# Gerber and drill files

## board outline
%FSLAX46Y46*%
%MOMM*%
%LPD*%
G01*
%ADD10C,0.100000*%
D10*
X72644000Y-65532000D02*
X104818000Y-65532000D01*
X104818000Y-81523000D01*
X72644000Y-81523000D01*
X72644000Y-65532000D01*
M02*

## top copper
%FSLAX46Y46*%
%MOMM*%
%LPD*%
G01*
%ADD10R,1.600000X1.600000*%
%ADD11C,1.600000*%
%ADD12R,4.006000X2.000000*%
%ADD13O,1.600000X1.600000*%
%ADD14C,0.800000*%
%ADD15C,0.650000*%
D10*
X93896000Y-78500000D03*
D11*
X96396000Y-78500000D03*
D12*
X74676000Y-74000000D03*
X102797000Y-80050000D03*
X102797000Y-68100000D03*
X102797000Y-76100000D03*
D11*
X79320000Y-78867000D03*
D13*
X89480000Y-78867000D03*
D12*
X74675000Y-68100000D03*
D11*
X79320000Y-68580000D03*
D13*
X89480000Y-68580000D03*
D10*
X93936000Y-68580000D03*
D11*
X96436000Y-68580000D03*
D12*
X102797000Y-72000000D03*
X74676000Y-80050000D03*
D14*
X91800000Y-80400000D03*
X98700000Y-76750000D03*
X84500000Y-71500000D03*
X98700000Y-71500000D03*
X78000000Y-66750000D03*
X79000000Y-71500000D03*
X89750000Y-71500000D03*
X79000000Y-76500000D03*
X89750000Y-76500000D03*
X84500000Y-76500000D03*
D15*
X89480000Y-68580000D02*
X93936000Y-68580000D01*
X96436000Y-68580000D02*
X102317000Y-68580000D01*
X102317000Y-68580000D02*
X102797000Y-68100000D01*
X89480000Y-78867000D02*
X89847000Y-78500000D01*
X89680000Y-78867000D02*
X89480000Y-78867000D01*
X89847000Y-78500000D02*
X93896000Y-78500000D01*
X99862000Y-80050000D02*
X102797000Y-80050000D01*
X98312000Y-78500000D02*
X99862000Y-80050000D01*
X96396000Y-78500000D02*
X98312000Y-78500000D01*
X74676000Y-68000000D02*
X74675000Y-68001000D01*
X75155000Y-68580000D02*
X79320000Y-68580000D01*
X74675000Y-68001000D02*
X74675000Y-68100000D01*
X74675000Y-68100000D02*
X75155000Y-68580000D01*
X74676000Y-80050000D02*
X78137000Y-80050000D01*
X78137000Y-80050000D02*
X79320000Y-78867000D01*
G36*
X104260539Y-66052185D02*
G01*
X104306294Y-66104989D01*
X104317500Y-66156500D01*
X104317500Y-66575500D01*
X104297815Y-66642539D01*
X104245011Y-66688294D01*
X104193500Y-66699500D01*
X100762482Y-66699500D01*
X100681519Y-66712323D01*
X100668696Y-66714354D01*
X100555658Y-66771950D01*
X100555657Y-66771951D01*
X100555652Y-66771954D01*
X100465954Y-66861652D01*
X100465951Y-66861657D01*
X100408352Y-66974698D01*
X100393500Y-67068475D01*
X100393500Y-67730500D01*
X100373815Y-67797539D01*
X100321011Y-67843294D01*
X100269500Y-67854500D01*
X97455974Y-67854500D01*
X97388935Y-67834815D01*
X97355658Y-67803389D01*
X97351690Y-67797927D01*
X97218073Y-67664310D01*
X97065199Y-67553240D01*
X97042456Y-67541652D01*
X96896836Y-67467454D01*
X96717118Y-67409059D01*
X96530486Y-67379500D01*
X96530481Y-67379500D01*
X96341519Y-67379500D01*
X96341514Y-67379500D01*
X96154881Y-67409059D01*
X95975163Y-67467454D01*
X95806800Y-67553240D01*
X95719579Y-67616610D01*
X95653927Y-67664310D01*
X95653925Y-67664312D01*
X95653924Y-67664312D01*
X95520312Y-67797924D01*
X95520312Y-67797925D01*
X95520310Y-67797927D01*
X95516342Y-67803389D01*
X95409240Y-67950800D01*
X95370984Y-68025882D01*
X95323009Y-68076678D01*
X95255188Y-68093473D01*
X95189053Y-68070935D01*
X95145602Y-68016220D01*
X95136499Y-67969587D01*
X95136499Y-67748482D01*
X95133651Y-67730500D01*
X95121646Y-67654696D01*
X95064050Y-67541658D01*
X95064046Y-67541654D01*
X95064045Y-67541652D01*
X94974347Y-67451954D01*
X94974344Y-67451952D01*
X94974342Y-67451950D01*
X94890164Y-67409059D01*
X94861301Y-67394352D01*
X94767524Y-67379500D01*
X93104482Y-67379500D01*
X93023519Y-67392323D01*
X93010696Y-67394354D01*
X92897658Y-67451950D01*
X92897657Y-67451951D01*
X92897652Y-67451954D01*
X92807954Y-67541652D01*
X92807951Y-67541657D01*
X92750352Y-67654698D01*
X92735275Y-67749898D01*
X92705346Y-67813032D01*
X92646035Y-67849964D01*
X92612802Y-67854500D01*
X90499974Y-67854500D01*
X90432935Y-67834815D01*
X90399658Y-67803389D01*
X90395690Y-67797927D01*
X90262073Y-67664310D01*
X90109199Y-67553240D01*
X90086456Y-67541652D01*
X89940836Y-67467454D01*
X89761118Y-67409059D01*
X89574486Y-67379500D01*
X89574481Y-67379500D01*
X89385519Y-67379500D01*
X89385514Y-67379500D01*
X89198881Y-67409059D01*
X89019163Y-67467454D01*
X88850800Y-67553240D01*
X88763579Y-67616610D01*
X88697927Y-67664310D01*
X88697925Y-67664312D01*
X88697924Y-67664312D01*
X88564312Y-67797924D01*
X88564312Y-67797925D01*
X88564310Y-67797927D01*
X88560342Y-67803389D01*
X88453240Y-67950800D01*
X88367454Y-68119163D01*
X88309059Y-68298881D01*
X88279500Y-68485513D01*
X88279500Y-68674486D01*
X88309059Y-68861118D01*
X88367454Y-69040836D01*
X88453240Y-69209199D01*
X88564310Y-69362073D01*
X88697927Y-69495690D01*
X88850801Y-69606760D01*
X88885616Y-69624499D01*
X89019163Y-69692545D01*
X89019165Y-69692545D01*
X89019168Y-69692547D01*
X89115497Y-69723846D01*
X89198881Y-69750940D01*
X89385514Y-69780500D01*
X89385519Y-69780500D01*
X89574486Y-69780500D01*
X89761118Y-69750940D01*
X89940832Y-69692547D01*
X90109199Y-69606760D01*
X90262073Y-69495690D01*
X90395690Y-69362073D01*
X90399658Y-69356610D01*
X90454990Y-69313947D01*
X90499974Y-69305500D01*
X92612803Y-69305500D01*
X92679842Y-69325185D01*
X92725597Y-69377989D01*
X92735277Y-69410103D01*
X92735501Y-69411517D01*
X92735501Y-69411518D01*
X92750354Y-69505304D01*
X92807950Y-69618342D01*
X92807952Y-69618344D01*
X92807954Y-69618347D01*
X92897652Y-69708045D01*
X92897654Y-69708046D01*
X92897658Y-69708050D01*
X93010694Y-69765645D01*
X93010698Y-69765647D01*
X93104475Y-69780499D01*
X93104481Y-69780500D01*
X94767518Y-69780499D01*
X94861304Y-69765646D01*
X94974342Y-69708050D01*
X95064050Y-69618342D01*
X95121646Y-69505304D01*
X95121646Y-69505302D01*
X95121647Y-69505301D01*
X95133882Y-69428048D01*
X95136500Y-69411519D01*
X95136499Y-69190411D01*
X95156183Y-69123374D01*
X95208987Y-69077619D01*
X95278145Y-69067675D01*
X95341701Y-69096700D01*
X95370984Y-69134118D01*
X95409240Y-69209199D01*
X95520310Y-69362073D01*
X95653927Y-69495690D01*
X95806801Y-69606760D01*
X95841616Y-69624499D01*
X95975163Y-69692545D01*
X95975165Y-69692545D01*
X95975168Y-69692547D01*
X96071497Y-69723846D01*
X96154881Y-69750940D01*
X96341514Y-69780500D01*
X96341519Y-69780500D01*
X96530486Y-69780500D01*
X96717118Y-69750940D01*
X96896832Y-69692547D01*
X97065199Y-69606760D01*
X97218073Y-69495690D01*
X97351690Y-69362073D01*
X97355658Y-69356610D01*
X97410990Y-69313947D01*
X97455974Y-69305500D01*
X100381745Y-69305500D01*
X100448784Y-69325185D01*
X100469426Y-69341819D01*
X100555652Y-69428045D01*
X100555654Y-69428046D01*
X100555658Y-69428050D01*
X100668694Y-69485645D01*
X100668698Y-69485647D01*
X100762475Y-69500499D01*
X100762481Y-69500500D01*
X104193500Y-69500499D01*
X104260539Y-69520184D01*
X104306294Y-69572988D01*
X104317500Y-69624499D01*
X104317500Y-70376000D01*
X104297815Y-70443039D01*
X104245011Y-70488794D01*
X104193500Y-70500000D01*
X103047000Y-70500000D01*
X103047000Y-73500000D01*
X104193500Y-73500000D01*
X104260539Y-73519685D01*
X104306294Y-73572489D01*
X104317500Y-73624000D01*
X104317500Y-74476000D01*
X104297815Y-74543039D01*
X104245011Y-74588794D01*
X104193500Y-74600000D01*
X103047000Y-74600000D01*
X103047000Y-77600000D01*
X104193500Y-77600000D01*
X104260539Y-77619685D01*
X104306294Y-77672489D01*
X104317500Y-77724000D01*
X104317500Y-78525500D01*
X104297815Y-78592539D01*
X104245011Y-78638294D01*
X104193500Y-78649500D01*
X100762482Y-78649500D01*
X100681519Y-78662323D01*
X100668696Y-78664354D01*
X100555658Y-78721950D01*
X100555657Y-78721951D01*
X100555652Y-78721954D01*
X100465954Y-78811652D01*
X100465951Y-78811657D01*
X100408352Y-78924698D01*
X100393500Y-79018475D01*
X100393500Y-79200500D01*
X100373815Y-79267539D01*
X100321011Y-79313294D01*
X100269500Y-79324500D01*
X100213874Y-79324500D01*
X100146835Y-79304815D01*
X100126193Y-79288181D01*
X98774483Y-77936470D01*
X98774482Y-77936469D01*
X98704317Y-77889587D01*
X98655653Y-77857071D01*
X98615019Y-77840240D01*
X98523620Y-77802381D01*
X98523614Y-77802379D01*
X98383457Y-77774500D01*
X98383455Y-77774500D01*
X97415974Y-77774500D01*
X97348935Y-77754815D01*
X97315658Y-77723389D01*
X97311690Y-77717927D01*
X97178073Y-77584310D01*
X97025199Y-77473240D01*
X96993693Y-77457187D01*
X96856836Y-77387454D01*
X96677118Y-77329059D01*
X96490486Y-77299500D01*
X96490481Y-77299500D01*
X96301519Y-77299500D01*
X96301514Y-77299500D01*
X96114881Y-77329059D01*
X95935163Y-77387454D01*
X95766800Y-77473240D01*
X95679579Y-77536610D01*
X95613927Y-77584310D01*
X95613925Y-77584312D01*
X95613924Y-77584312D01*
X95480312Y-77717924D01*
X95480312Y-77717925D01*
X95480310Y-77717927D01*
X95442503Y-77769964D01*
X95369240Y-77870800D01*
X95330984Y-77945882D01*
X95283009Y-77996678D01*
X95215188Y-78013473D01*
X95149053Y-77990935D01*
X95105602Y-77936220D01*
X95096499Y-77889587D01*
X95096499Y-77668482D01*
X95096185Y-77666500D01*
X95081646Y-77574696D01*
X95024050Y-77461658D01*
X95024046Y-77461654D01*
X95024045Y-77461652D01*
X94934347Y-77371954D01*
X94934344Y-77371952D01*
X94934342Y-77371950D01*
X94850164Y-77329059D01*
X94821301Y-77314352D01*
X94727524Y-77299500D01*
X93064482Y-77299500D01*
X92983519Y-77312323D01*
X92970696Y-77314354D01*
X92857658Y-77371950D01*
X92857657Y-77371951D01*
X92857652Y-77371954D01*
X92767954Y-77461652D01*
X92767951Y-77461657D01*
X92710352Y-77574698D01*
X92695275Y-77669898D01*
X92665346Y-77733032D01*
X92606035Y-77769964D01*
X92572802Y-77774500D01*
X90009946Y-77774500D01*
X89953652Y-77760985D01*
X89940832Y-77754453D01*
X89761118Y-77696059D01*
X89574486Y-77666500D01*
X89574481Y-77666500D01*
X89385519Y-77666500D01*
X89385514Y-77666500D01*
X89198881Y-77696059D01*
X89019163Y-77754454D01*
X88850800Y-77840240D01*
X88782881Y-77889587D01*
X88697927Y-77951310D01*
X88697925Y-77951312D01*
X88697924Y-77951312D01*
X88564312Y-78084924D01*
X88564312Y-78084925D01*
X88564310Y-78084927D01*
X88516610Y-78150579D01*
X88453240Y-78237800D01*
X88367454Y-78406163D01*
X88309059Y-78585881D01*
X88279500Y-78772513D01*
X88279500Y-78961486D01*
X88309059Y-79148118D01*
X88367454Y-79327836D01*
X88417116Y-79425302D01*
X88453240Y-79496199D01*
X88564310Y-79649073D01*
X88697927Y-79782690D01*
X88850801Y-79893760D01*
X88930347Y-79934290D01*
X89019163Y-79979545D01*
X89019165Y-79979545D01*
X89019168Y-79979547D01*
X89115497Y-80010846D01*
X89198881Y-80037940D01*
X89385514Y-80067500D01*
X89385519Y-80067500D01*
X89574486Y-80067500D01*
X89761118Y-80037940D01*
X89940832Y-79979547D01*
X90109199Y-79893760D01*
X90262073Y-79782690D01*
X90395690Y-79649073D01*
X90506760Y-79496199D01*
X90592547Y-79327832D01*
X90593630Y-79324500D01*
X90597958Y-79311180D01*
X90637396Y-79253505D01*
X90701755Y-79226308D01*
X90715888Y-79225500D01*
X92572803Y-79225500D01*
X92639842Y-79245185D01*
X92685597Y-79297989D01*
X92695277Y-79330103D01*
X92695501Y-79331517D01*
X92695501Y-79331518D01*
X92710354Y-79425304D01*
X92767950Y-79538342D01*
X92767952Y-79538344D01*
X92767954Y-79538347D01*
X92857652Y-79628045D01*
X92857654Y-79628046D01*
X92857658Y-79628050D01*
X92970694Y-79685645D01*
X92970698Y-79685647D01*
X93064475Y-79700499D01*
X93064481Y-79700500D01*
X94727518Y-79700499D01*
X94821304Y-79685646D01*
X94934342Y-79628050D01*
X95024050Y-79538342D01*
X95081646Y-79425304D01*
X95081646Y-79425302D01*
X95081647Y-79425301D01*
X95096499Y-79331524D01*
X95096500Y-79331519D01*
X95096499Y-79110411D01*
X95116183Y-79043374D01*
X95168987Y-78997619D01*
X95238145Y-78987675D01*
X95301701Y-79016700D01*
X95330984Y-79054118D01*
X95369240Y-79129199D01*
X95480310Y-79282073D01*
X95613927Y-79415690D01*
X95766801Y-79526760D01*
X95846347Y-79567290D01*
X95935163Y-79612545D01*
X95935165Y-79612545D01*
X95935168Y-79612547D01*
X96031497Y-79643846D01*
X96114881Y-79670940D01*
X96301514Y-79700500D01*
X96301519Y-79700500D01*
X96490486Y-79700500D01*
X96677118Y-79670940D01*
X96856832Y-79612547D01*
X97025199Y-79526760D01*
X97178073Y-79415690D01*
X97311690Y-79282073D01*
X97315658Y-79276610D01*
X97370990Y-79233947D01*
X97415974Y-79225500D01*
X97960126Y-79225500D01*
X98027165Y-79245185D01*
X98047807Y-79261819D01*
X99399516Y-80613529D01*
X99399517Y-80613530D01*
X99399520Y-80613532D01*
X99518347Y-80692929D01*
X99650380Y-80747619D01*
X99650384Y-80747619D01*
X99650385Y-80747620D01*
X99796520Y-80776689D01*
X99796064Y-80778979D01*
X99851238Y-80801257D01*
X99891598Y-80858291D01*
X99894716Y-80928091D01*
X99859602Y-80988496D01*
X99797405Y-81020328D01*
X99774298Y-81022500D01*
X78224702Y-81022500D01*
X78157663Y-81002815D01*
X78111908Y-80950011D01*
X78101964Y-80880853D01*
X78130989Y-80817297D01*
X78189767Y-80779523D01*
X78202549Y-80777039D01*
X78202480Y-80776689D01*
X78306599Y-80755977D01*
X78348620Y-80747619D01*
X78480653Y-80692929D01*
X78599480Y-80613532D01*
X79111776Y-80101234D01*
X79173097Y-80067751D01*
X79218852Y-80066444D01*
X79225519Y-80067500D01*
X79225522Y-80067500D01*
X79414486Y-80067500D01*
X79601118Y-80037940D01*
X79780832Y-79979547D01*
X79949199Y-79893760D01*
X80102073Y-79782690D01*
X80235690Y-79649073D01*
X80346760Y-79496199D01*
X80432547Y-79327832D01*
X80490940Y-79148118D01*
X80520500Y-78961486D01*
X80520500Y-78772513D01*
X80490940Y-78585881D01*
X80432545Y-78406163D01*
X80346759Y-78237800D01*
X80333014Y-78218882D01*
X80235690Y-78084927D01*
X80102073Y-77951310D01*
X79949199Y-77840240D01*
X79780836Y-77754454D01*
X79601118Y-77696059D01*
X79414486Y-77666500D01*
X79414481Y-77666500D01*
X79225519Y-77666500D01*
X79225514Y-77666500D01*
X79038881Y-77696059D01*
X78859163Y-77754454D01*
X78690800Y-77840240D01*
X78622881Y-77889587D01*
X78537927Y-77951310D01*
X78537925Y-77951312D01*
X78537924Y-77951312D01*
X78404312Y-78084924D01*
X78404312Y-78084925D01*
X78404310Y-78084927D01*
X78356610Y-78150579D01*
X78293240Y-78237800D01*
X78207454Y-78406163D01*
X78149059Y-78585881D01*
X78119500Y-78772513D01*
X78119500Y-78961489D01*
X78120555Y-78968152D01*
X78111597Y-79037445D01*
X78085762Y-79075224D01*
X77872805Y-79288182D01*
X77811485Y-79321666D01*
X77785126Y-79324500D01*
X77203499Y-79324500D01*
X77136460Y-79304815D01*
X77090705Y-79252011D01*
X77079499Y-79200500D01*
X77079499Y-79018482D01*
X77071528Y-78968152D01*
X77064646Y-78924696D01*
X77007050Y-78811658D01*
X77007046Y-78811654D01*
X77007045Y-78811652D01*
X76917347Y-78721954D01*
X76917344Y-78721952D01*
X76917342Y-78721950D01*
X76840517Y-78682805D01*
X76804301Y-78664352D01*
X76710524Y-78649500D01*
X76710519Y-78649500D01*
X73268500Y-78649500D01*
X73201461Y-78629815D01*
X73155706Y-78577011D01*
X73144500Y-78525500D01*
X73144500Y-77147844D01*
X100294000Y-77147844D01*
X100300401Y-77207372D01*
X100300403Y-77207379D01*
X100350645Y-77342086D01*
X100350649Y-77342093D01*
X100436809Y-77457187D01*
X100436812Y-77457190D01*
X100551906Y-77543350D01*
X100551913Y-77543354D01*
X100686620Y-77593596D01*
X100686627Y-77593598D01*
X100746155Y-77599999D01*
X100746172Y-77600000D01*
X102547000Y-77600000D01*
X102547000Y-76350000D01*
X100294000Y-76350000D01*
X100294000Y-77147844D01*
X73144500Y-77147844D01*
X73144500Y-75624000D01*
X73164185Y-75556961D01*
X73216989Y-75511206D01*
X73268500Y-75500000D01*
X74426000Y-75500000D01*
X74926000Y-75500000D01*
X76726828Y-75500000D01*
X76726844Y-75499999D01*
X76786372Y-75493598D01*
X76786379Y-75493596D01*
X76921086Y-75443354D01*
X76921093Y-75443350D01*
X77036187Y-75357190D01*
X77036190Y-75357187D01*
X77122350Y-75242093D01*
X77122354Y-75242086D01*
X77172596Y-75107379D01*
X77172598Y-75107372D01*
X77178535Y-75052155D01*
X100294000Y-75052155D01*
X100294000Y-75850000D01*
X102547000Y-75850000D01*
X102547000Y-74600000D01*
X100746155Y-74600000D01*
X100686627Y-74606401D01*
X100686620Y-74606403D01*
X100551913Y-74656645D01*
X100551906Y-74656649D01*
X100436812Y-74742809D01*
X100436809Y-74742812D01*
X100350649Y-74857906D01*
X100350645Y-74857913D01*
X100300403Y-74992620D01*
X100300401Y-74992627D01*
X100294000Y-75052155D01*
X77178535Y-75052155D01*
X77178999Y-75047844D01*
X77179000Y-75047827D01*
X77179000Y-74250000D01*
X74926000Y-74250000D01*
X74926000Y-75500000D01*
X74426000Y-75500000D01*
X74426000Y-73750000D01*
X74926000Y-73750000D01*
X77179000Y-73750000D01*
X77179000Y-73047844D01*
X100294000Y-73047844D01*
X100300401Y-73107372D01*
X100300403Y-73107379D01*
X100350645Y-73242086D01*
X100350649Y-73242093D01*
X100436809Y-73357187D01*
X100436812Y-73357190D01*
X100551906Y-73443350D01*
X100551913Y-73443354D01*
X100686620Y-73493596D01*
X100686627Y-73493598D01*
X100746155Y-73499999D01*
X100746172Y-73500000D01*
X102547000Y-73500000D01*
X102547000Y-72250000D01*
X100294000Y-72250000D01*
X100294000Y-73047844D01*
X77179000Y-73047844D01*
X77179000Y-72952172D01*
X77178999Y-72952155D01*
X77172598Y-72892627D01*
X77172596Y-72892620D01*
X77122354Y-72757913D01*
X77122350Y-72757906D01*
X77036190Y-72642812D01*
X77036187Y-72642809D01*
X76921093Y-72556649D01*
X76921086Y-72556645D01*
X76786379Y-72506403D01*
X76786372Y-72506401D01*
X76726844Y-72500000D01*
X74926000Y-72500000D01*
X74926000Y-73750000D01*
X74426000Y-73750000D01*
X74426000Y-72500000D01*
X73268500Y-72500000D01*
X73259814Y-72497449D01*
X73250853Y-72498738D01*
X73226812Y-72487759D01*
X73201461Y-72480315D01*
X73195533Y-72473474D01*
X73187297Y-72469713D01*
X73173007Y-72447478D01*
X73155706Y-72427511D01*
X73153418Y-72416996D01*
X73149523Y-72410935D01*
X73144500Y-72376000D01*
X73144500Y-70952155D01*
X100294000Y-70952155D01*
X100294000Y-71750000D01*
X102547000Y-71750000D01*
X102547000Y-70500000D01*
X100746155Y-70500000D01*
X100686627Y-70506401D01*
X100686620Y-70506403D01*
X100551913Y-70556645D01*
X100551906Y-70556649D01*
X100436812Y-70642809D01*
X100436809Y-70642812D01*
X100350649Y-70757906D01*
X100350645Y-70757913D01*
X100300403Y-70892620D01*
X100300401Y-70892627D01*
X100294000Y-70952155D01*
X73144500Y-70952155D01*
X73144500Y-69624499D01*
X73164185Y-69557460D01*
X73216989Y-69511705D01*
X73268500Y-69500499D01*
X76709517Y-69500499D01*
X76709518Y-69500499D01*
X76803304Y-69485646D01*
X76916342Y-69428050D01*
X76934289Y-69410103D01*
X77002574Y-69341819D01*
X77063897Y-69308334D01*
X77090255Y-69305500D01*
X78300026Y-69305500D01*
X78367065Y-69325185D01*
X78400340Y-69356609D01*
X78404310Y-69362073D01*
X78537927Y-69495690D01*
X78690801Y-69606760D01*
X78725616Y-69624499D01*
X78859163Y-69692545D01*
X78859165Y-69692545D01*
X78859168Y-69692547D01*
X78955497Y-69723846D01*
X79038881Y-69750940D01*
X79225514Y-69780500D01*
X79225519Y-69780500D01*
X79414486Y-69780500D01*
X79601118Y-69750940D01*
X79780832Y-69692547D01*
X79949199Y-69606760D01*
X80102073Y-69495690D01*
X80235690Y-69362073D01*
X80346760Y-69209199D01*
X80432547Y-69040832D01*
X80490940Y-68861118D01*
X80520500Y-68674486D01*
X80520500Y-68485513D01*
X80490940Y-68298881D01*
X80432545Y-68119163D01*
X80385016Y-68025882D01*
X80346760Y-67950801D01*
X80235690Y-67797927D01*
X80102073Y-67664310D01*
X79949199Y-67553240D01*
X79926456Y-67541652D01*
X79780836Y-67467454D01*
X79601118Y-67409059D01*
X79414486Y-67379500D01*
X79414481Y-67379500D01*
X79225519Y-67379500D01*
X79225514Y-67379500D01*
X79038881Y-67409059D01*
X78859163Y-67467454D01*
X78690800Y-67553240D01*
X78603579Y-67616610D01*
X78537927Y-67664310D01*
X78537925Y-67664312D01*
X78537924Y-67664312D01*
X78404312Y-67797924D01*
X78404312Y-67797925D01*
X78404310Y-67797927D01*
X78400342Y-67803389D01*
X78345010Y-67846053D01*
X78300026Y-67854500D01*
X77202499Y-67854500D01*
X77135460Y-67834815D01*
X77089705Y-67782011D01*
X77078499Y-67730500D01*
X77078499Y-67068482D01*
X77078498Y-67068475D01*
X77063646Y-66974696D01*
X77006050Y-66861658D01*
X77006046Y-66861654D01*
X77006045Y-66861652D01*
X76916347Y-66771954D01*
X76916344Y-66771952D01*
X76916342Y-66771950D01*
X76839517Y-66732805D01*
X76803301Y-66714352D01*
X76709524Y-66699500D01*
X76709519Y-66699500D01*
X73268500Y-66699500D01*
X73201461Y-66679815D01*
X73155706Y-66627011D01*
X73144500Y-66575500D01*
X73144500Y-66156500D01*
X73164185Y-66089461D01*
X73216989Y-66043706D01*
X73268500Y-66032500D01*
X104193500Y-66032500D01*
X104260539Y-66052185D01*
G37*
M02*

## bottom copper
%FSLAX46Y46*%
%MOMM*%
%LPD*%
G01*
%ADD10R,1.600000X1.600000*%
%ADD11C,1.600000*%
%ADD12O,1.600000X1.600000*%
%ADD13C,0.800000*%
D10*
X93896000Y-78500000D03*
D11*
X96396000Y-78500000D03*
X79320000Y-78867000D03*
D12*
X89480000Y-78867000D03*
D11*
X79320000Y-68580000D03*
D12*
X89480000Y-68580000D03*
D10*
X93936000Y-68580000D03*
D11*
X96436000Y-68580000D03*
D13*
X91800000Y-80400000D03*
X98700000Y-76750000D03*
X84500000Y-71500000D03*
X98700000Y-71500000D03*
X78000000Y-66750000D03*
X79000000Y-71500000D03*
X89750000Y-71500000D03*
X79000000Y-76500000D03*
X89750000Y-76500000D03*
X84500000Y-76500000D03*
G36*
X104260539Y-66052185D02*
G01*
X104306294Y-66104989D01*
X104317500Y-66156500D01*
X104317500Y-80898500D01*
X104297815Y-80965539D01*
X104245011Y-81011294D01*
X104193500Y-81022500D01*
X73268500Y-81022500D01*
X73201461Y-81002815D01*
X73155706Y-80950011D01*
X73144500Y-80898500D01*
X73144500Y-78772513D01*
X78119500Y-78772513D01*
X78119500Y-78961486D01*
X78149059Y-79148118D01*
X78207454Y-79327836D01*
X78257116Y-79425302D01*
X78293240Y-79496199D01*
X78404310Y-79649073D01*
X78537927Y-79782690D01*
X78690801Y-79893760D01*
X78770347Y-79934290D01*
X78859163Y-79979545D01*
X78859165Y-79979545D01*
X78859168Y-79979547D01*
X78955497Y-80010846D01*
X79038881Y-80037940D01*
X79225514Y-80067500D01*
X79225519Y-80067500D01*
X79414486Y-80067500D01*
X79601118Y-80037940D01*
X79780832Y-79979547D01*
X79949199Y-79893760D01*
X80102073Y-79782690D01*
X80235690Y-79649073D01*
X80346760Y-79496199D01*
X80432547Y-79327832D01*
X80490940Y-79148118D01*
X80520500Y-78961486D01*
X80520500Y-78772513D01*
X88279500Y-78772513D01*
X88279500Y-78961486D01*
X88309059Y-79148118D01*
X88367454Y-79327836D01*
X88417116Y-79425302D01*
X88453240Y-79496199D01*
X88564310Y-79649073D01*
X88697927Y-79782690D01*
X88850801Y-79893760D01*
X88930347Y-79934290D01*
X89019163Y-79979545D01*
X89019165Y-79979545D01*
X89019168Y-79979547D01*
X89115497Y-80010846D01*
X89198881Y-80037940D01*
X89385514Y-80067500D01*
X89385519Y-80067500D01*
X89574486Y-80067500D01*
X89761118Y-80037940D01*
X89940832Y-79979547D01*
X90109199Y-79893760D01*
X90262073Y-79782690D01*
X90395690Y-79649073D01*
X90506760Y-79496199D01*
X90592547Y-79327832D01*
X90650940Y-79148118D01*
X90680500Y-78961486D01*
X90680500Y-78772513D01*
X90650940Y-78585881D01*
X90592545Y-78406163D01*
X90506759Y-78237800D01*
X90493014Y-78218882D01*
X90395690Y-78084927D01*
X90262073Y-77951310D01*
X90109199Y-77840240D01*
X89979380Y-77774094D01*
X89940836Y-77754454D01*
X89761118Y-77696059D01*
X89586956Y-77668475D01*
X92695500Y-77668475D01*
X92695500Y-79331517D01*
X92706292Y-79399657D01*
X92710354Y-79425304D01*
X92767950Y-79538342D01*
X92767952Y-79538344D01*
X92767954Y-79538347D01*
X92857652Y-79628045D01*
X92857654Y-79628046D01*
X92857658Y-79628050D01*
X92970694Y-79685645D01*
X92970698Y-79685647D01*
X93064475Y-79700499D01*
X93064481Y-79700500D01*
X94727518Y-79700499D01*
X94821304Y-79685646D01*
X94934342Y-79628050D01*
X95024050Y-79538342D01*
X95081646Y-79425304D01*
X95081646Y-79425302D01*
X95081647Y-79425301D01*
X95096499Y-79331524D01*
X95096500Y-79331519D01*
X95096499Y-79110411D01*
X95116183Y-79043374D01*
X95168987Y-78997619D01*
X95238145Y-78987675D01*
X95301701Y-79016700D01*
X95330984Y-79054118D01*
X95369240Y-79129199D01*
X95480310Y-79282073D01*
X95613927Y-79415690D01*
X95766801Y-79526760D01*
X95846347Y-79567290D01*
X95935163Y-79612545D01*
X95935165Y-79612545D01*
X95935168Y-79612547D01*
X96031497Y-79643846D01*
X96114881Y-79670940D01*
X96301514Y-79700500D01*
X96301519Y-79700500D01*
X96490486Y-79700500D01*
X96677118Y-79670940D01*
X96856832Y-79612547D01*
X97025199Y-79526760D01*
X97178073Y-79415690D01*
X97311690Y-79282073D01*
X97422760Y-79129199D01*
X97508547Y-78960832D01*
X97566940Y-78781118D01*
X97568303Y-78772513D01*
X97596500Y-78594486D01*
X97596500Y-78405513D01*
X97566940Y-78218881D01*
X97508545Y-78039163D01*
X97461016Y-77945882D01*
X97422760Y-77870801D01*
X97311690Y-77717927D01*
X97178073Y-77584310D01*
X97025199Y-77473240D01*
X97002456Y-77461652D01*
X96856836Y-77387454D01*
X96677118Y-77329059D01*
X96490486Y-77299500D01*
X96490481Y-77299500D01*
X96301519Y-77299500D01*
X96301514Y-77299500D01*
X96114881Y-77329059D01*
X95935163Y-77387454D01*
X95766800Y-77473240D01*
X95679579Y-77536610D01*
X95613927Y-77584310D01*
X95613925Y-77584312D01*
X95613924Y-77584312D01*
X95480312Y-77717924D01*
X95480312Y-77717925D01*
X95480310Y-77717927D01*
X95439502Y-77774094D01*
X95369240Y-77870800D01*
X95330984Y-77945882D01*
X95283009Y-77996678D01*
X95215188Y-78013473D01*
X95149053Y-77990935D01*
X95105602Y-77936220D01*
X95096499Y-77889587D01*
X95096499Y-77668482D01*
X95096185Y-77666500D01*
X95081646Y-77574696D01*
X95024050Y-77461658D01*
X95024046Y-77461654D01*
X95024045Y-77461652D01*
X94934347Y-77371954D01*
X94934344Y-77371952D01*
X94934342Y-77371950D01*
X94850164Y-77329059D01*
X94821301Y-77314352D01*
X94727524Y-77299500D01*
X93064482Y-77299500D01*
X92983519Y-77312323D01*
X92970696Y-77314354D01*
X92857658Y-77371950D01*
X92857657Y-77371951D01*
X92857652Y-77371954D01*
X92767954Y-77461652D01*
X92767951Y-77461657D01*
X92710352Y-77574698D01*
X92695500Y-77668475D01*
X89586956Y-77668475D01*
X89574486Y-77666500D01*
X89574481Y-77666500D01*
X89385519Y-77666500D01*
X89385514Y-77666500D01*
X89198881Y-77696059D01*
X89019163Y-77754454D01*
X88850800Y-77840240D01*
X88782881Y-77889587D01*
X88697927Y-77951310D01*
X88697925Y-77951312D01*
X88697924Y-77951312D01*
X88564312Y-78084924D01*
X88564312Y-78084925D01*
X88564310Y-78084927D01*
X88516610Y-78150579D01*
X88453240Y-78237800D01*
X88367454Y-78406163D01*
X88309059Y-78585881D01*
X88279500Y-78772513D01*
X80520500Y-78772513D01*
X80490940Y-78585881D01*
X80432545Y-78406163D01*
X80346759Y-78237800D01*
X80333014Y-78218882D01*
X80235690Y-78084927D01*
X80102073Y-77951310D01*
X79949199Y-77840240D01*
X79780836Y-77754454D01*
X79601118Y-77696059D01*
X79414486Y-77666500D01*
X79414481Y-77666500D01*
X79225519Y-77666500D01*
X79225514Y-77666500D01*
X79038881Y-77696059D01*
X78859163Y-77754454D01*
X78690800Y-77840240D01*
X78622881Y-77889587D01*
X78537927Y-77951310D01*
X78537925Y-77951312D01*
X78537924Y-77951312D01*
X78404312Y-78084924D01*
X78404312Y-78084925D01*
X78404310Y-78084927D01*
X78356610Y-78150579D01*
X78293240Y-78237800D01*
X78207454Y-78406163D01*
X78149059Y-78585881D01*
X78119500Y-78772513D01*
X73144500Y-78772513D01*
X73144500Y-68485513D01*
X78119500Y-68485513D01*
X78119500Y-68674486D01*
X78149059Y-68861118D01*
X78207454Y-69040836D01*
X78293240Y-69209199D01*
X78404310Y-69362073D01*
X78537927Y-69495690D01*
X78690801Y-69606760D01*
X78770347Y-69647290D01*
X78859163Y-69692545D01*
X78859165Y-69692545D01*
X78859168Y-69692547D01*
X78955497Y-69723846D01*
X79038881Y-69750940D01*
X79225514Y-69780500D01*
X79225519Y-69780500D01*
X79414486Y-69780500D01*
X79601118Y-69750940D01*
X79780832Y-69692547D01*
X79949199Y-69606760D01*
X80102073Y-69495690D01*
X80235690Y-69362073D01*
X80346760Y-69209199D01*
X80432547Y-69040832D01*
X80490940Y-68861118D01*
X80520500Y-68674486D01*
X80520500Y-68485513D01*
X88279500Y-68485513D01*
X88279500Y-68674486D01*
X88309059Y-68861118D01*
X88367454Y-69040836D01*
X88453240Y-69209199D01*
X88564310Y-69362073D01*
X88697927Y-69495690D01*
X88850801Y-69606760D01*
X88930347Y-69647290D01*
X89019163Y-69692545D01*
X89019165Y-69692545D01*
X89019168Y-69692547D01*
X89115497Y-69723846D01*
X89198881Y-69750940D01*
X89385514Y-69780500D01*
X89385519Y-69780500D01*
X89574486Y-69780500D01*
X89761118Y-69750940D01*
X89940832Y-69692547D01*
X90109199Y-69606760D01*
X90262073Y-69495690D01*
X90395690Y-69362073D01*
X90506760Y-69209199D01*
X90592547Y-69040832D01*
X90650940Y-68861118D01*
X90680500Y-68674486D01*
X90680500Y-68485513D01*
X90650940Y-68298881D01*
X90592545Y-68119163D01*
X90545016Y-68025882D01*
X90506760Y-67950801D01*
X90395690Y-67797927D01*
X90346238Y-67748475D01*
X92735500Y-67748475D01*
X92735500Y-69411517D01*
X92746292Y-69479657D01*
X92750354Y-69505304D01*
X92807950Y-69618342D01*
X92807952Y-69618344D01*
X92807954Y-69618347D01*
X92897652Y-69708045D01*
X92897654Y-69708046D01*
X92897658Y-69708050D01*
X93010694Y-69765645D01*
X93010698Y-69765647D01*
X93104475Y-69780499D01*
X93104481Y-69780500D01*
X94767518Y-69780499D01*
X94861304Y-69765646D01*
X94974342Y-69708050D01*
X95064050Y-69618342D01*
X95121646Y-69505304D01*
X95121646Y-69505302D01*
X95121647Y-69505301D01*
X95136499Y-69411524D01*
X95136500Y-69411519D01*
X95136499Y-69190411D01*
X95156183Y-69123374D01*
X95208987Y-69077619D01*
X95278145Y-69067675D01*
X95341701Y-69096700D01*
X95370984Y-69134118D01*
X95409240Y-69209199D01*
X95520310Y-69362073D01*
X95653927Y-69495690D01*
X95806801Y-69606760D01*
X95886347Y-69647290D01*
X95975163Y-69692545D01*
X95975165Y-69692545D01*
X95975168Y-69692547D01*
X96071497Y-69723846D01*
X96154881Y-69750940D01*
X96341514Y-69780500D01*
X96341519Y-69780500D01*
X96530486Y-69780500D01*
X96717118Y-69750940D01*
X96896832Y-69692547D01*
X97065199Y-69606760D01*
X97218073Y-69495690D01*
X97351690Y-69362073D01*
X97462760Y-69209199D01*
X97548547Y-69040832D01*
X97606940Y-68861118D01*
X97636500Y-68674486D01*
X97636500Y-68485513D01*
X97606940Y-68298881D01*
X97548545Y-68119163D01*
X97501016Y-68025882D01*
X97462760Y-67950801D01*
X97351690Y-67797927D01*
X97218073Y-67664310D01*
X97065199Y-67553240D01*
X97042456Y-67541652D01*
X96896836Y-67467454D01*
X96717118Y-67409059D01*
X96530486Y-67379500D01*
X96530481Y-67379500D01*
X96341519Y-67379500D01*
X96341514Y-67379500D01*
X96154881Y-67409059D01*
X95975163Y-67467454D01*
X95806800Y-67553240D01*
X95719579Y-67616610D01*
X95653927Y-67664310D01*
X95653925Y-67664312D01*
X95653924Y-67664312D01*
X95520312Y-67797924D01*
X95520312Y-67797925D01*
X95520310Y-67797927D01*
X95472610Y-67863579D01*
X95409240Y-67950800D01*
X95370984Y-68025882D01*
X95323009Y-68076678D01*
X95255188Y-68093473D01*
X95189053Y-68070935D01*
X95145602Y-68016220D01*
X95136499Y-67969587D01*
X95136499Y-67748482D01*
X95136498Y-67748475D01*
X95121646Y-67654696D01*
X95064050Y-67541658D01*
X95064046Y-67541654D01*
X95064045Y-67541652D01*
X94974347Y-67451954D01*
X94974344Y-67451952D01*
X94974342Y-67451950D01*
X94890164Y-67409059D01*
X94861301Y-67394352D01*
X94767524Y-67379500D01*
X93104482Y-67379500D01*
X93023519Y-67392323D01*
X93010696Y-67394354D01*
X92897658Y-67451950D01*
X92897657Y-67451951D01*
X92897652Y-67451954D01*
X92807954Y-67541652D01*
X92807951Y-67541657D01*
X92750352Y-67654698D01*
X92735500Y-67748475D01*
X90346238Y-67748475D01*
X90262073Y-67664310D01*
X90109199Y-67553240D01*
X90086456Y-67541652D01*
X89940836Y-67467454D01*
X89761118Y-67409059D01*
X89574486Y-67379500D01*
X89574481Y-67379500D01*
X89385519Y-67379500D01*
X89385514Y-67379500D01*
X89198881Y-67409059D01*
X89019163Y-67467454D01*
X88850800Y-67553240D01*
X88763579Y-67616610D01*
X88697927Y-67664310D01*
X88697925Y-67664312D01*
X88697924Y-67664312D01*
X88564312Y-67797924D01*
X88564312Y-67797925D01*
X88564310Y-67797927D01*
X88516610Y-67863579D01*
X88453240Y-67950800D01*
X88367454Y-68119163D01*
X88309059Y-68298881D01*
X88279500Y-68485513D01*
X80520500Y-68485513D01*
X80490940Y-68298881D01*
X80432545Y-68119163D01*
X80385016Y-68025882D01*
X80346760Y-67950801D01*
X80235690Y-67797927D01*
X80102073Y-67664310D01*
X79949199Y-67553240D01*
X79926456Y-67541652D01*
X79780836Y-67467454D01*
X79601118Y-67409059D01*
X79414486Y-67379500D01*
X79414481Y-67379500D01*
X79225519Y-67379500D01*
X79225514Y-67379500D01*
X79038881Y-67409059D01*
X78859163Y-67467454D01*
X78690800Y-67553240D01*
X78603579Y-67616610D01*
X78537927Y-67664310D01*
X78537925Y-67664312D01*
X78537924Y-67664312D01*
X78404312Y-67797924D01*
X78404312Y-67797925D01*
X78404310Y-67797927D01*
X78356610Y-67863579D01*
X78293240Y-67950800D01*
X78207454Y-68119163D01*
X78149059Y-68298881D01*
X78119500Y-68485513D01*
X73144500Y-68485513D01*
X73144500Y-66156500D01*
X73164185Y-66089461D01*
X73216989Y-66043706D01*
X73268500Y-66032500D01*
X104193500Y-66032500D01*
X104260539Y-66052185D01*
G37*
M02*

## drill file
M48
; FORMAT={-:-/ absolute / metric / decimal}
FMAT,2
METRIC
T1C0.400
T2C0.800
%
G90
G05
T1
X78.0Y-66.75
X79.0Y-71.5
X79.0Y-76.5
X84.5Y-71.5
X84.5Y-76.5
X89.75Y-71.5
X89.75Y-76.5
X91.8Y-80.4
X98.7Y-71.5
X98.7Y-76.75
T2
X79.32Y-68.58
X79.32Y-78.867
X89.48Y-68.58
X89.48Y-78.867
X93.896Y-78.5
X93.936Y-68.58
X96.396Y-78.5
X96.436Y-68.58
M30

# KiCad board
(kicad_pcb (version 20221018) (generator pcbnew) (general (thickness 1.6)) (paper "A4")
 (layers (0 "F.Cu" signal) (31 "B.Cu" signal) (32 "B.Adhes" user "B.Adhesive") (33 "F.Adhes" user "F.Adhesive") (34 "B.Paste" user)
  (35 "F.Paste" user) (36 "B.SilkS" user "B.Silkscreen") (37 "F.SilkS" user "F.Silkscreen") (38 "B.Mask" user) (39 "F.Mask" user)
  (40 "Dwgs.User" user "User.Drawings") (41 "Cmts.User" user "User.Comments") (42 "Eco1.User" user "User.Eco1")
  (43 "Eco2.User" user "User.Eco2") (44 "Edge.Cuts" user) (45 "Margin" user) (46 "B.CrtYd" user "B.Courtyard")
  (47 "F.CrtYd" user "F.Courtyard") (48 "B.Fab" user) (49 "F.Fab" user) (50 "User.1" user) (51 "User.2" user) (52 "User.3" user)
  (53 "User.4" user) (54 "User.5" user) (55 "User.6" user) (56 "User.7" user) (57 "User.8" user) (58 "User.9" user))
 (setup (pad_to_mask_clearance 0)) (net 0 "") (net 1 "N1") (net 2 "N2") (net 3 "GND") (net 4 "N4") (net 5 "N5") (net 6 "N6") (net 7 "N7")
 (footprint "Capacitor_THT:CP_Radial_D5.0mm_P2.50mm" (layer "F.Cu") (at 93.896 78.5)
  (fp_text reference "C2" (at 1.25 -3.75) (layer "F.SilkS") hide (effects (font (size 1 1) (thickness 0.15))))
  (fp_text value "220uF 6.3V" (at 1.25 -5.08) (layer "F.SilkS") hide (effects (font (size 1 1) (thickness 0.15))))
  (pad "1" thru_hole rect (at 0 0) (size 1.6 1.6) (drill 0.8) (layers "*.Cu" "*.Mask") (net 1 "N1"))
  (pad "2" thru_hole circle (at 2.5 0) (size 1.6 1.6) (drill 0.8) (layers "*.Cu" "*.Mask") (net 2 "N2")))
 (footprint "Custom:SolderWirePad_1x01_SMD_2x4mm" (layer "F.Cu") (at 74.673 74 -90)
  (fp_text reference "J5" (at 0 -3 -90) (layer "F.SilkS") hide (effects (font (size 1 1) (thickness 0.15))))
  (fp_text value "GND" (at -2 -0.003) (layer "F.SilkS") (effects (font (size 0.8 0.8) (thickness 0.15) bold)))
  (pad "1" smd rect (at 0 -0.003 270) (size 2 4.006) (layers "F.Cu" "F.Paste" "F.Mask") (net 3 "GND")))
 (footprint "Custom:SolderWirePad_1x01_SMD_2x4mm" (layer "F.Cu") (at 102.8 80.05 90)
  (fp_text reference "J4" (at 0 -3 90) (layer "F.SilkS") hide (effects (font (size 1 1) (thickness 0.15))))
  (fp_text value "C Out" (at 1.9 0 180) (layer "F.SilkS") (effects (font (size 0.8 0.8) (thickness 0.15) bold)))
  (pad "1" smd rect (at 0 -0.003 90) (size 2 4.006) (layers "F.Cu" "F.Paste" "F.Mask") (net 2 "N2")))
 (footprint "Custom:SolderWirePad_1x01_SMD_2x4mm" (layer "F.Cu") (at 102.8 68.1 90)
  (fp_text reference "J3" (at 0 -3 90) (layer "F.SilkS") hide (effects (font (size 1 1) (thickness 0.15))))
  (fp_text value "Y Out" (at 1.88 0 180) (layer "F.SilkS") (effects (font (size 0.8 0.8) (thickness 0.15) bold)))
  (pad "1" smd rect (at 0 -0.003 90) (size 2 4.006) (layers "F.Cu" "F.Paste" "F.Mask") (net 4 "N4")))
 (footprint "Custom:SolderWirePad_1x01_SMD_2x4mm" (layer "F.Cu") (at 102.8 76.1 90)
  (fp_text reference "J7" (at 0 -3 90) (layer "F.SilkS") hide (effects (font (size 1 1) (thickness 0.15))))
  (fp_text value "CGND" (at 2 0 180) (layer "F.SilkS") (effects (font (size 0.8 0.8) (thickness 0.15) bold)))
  (pad "1" smd rect (at 0 -0.003 90) (size 2 4.006) (layers "F.Cu" "F.Paste" "F.Mask") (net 3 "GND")))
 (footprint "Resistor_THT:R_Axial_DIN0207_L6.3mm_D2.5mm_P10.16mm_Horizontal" (layer "F.Cu") (at 79.32 78.867)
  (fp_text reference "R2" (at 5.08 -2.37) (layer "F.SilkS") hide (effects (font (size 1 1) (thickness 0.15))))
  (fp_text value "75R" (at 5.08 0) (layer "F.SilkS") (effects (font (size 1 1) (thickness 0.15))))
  (pad "1" thru_hole circle (at 0 0) (size 1.6 1.6) (drill 0.8) (layers "*.Cu" "*.Mask") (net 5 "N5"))
  (pad "2" thru_hole oval (at 10.16 0) (size 1.6 1.6) (drill 0.8) (layers "*.Cu" "*.Mask") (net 1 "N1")))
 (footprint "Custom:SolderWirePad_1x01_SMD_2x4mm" (layer "F.Cu") (at 74.672 68.1 -90)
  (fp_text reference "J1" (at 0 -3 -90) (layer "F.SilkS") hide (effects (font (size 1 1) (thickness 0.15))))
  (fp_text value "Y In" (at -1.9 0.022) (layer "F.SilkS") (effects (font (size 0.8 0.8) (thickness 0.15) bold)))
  (pad "1" smd rect (at 0 -0.003 270) (size 2 4.006) (layers "F.Cu" "F.Paste" "F.Mask") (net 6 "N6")))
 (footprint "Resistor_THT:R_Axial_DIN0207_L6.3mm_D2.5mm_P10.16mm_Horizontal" (layer "F.Cu") (at 79.32 68.58)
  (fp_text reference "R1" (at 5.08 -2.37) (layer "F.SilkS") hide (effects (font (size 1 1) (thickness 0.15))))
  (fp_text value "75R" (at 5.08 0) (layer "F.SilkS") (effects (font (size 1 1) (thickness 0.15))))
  (pad "1" thru_hole circle (at 0 0) (size 1.6 1.6) (drill 0.8) (layers "*.Cu" "*.Mask") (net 6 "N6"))
  (pad "2" thru_hole oval (at 10.16 0) (size 1.6 1.6) (drill 0.8) (layers "*.Cu" "*.Mask") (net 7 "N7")))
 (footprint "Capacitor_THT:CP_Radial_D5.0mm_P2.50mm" (layer "F.Cu") (at 93.936 68.58)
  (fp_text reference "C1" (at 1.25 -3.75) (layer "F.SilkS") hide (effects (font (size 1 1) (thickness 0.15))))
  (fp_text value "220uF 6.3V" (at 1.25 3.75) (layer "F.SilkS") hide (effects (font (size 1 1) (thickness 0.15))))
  (pad "1" thru_hole rect (at 0 0) (size 1.6 1.6) (drill 0.8) (layers "*.Cu" "*.Mask") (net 7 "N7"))
  (pad "2" thru_hole circle (at 2.5 0) (size 1.6 1.6) (drill 0.8) (layers "*.Cu" "*.Mask") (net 4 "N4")))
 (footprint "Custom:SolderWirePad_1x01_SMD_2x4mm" (layer "F.Cu") (at 102.8 72 90)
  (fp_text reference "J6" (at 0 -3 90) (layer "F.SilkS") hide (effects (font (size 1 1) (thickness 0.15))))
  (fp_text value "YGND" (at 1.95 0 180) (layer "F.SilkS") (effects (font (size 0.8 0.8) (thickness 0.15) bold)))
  (pad "1" smd rect (at 0 -0.003 90) (size 2 4.006) (layers "F.Cu" "F.Paste" "F.Mask") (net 3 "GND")))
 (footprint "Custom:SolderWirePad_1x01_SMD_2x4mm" (layer "F.Cu") (at 74.673 80.05 -90)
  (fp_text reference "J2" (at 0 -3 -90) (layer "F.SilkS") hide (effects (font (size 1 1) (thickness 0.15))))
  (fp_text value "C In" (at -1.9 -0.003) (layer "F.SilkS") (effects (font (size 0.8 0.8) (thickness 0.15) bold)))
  (pad "1" smd rect (at 0 -0.003 270) (size 2 4.006) (layers "F.Cu" "F.Paste" "F.Mask") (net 5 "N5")))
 (gr_rect (start 72.644 65.532) (end 104.818 81.523) (stroke (width 0.1) (type default)) (fill none) (layer "Edge.Cuts"))
 (segment (start 89.48 68.58) (end 93.936 68.58) (width 0.65) (layer "F.Cu") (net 7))
 (segment (start 96.436 68.58) (end 102.317 68.58) (width 0.65) (layer "F.Cu") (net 4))
 (segment (start 102.317 68.58) (end 102.797 68.1) (width 0.65) (layer "F.Cu") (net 4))
 (segment (start 89.48 78.867) (end 89.847 78.5) (width 0.65) (layer "F.Cu") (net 1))
 (segment (start 89.68 78.867) (end 89.48 78.867) (width 0.65) (layer "F.Cu") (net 1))
 (segment (start 89.847 78.5) (end 93.896 78.5) (width 0.65) (layer "F.Cu") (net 1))
 (segment (start 99.862 80.05) (end 102.797 80.05) (width 0.65) (layer "F.Cu") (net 2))
 (segment (start 98.312 78.5) (end 99.862 80.05) (width 0.65) (layer "F.Cu") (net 2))
 (segment (start 96.396 78.5) (end 98.312 78.5) (width 0.65) (layer "F.Cu") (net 2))
 (segment (start 74.676 68) (end 74.675 68.001) (width 0.65) (layer "F.Cu") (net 6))
 (segment (start 75.155 68.58) (end 79.32 68.58) (width 0.65) (layer "F.Cu") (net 6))
 (segment (start 74.675 68.001) (end 74.675 68.1) (width 0.65) (layer "F.Cu") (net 6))
 (segment (start 74.675 68.1) (end 75.155 68.58) (width 0.65) (layer "F.Cu") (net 6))
 (segment (start 74.676 80.05) (end 78.137 80.05) (width 0.65) (layer "F.Cu") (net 5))
 (segment (start 78.137 80.05) (end 79.32 78.867) (width 0.65) (layer "F.Cu") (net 5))
 (via (at 91.8 80.4) (size 0.8) (drill 0.4) (layers "F.Cu" "B.Cu") (free) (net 3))
 (via (at 98.7 76.75) (size 0.8) (drill 0.4) (layers "F.Cu" "B.Cu") (free) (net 3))
 (via (at 84.5 71.5) (size 0.8) (drill 0.4) (layers "F.Cu" "B.Cu") (free) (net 3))
 (via (at 98.7 71.5) (size 0.8) (drill 0.4) (layers "F.Cu" "B.Cu") (free) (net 3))
 (via (at 78 66.75) (size 0.8) (drill 0.4) (layers "F.Cu" "B.Cu") (free) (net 3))
 (via (at 79 71.5) (size 0.8) (drill 0.4) (layers "F.Cu" "B.Cu") (free) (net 3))
 (via (at 89.75 71.5) (size 0.8) (drill 0.4) (layers "F.Cu" "B.Cu") (free) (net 3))
 (via (at 79 76.5) (size 0.8) (drill 0.4) (layers "F.Cu" "B.Cu") (free) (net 3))
 (via (at 89.75 76.5) (size 0.8) (drill 0.4) (layers "F.Cu" "B.Cu") (free) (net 3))
 (via (at 84.5 76.5) (size 0.8) (drill 0.4) (layers "F.Cu" "B.Cu") (free) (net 3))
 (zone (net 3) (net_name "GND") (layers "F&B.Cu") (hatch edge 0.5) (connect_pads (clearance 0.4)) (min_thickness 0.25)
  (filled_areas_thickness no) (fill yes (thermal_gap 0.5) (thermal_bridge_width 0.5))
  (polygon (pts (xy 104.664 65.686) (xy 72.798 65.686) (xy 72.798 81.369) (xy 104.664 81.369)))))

